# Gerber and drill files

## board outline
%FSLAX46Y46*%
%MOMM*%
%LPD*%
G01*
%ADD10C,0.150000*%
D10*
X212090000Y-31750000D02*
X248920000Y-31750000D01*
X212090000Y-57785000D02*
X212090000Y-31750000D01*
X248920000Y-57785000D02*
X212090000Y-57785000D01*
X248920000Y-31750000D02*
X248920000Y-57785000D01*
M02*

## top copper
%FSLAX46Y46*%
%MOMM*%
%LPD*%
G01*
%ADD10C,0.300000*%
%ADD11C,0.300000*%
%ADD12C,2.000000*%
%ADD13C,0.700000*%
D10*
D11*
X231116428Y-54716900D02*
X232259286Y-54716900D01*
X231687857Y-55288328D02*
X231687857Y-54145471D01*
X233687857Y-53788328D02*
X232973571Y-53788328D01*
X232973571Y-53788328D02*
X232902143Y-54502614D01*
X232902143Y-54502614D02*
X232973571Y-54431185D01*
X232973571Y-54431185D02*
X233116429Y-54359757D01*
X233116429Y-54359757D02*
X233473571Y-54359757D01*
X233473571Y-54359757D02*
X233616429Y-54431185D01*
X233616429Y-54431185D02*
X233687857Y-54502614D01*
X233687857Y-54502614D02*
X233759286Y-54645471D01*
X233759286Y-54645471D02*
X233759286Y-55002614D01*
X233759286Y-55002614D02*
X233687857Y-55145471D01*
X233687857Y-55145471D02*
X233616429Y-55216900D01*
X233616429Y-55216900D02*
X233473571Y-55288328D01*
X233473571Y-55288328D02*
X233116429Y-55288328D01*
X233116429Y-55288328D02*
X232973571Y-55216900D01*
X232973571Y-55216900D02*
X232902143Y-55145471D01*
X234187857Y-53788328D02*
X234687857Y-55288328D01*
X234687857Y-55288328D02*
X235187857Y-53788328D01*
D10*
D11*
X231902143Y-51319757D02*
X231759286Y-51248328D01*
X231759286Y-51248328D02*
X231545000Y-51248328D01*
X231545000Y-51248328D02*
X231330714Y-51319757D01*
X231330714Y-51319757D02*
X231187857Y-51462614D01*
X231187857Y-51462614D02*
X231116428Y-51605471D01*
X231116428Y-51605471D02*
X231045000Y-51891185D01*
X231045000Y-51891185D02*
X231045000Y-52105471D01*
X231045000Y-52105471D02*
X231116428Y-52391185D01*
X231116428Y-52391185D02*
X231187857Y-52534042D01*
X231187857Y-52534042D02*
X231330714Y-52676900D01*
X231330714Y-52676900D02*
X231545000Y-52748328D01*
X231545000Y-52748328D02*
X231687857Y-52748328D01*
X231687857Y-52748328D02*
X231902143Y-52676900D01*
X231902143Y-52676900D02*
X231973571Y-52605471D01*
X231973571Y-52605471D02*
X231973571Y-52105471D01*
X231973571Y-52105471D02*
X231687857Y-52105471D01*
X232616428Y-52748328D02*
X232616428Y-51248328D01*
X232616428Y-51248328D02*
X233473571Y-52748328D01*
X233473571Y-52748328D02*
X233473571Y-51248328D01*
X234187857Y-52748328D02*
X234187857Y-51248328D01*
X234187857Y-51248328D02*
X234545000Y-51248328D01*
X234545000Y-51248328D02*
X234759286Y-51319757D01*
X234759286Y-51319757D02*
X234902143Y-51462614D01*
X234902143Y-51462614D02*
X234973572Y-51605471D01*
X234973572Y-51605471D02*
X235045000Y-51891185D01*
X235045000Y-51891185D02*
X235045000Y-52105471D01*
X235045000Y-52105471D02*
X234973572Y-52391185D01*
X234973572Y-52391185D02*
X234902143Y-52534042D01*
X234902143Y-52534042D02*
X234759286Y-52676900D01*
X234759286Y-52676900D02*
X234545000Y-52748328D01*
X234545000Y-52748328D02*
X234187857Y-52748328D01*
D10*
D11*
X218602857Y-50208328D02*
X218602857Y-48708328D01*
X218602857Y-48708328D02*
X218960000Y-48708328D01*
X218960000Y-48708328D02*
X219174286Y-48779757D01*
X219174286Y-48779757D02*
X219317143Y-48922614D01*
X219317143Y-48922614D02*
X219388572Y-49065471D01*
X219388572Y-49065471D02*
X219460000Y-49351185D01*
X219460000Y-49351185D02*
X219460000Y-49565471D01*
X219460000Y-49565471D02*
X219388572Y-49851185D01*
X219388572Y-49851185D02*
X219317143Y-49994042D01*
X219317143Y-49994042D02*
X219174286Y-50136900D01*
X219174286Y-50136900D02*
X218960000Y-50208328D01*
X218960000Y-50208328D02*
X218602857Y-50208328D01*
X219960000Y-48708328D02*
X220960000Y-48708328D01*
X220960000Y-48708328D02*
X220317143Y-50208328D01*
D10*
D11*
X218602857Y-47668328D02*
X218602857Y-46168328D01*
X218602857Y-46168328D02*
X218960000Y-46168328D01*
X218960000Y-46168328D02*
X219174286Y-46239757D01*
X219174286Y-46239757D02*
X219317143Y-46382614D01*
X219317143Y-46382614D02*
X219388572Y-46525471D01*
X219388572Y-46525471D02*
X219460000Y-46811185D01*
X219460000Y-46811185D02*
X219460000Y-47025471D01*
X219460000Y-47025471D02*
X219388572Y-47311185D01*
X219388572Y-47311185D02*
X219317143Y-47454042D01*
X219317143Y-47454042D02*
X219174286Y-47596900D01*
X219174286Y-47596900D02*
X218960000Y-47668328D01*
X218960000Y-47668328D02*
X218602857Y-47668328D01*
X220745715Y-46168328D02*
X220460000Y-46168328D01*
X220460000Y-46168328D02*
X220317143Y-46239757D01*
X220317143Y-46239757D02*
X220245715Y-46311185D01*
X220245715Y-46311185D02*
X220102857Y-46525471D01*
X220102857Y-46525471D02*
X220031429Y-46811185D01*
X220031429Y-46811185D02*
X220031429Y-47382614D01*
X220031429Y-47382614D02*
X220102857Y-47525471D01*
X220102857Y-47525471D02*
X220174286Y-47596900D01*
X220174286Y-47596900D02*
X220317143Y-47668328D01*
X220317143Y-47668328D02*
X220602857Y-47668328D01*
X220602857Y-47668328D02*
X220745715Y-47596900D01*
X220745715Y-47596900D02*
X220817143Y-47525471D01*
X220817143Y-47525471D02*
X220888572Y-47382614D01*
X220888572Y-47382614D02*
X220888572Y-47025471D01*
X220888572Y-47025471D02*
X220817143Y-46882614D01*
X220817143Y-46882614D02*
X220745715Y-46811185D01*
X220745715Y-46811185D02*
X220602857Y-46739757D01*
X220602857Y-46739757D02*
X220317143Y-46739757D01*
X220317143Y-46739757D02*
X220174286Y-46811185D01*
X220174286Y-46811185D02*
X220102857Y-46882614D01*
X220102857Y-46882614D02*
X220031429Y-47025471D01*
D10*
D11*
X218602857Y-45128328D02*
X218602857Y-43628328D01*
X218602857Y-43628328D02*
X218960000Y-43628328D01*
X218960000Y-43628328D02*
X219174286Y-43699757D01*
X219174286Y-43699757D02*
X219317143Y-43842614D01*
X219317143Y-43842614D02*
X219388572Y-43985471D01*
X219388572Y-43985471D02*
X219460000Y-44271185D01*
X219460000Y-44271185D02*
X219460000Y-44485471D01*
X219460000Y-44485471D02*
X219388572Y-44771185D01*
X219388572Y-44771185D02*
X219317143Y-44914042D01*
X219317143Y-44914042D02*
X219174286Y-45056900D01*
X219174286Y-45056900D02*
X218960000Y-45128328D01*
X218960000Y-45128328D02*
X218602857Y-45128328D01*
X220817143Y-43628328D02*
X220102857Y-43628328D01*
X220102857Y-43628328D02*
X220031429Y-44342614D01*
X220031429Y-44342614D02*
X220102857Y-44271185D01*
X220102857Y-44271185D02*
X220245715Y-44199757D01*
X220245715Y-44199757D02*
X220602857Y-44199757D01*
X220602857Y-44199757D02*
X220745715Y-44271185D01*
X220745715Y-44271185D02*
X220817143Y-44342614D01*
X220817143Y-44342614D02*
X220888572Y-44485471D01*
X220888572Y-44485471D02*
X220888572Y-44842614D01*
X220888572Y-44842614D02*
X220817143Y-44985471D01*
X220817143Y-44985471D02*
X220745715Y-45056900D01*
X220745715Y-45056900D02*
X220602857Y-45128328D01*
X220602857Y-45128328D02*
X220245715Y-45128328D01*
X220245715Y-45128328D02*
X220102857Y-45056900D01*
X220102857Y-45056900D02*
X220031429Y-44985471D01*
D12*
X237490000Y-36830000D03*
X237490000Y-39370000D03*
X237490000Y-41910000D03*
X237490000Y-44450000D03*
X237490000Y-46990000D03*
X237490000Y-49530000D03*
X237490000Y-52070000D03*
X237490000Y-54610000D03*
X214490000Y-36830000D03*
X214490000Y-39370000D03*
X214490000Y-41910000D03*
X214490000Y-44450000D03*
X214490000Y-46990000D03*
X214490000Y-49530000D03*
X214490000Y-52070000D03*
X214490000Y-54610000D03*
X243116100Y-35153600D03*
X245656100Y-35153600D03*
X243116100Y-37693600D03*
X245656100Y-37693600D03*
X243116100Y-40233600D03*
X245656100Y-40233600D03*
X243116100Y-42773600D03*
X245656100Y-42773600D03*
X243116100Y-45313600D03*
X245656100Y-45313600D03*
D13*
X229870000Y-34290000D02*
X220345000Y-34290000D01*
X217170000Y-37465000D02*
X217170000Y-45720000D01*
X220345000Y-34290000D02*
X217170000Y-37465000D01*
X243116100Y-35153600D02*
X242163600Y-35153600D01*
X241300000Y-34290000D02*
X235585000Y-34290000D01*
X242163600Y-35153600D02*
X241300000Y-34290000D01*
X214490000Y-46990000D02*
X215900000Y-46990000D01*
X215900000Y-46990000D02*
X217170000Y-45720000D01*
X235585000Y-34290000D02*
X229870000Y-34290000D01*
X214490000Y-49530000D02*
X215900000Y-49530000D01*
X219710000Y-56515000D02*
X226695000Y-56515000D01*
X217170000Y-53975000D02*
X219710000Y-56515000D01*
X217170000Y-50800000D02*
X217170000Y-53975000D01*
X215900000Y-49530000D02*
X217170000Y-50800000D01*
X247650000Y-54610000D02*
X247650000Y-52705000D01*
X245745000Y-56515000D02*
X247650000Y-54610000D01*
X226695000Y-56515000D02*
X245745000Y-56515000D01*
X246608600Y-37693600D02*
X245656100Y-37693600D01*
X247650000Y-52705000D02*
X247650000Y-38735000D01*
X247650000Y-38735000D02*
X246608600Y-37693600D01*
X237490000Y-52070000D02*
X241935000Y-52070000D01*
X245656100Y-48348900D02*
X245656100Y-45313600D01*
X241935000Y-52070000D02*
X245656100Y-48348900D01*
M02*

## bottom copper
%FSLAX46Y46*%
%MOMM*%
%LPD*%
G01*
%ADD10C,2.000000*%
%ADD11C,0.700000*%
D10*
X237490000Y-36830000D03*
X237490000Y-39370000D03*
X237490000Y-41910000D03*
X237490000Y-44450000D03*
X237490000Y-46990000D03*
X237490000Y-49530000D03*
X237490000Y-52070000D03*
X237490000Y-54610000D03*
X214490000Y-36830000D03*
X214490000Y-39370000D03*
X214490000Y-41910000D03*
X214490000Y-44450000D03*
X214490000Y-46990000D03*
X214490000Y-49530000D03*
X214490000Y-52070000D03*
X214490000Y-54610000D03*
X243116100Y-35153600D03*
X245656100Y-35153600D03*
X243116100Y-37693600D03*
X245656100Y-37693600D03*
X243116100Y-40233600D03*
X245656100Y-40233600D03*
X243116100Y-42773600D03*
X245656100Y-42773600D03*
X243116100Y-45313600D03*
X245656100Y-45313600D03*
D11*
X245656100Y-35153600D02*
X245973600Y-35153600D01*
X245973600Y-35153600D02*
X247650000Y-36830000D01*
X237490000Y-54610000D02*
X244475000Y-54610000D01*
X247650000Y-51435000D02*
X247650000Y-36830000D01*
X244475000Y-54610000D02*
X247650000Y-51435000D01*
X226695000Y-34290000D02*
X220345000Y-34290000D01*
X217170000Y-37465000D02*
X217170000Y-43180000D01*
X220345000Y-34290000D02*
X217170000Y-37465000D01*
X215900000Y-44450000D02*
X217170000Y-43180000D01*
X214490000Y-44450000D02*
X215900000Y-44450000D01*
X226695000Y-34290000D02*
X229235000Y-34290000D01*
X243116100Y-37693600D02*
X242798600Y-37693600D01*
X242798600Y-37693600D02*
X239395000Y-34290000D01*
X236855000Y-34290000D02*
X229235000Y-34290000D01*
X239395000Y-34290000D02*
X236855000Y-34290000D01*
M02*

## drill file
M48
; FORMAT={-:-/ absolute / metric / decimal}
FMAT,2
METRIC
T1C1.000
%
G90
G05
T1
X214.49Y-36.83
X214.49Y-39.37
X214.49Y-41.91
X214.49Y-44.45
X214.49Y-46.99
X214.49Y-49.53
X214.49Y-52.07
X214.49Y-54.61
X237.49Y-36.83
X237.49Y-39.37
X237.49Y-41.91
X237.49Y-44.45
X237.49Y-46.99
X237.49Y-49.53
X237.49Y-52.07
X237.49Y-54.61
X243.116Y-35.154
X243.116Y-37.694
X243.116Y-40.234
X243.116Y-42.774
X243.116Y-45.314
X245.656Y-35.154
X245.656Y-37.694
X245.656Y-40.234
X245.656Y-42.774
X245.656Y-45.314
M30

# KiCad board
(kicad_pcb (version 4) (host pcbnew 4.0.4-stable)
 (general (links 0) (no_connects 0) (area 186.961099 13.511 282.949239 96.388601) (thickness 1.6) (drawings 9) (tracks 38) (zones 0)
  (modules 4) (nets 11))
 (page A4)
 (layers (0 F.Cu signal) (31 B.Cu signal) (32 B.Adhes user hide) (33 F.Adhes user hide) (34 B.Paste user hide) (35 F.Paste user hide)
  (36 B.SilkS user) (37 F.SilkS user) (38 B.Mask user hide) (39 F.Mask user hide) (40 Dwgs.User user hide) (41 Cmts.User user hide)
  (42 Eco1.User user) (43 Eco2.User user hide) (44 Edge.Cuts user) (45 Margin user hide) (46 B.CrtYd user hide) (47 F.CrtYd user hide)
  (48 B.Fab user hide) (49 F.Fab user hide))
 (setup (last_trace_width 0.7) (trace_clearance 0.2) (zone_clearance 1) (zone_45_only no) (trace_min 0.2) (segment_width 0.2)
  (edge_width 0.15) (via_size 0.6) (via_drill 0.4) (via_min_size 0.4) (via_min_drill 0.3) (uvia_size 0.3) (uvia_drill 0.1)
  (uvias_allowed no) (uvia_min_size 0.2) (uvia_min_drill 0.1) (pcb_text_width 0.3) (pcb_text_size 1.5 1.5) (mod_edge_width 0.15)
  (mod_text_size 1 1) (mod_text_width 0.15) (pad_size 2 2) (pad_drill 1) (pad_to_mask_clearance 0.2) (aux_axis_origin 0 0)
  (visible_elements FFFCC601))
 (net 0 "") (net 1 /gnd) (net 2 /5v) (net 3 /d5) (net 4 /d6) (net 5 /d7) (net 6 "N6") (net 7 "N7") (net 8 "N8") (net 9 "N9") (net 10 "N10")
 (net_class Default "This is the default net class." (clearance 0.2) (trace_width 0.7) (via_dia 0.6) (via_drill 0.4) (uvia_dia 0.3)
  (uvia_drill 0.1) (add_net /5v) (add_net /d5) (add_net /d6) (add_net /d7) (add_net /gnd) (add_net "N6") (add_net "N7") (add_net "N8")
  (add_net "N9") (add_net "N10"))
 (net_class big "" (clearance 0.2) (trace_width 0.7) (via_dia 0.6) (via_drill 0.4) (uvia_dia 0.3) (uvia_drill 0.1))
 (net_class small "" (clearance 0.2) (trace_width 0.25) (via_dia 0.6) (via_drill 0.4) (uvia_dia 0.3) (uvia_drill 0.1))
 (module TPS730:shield (layer F.Cu) (at 237.49 36.83)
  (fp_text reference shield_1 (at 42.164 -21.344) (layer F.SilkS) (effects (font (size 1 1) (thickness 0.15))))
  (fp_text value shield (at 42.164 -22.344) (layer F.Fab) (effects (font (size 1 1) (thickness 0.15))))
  (pad 14 thru_hole circle (at 0 0) (size 2 2) (drill 1) (layers *.Cu *.Mask))
  (pad 13 thru_hole circle (at 0 2.54) (size 2 2) (drill 1) (layers *.Cu *.Mask))
  (pad 12 thru_hole circle (at 0 5.08) (size 2 2) (drill 1) (layers *.Cu *.Mask))
  (pad 8 thru_hole circle (at 0 7.62) (size 2 2) (drill 1) (layers *.Cu *.Mask))
  (pad 7 thru_hole circle (at 0 10.16) (size 2 2) (drill 1) (layers *.Cu *.Mask))
  (pad 6 thru_hole circle (at 0 12.7) (size 2 2) (drill 1) (layers *.Cu *.Mask))
  (pad 5 thru_hole circle (at 0 15.24) (size 2 2) (drill 1) (layers *.Cu *.Mask) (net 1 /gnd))
  (pad 1 thru_hole circle (at 0 17.78) (size 2 2) (drill 1) (layers *.Cu *.Mask) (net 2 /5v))
  (pad 9 thru_hole circle (at -23 0) (size 2 2) (drill 1) (layers *.Cu *.Mask))
  (pad 10 thru_hole circle (at -23 2.54) (size 2 2) (drill 1) (layers *.Cu *.Mask))
  (pad 11 thru_hole circle (at -23 5.08) (size 2 2) (drill 1) (layers *.Cu *.Mask))
  (pad 4 thru_hole circle (at -23 7.62) (size 2 2) (drill 1) (layers *.Cu *.Mask) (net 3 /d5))
  (pad 3 thru_hole circle (at -23 10.16) (size 2 2) (drill 1) (layers *.Cu *.Mask) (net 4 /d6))
  (pad 2 thru_hole circle (at -23 12.7) (size 2 2) (drill 1) (layers *.Cu *.Mask) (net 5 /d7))
  (pad 15 thru_hole circle (at -23 15.24) (size 2 2) (drill 1) (layers *.Cu *.Mask))
  (pad 16 thru_hole circle (at -23 17.78) (size 2 2) (drill 1) (layers *.Cu *.Mask)))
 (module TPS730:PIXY (layer F.Cu) (at 250.7361 30.0736)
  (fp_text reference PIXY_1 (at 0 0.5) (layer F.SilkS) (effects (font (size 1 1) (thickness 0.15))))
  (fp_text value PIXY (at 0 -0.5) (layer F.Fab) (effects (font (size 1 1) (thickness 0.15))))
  (pad 1 thru_hole circle (at -7.62 5.08) (size 2 2) (drill 1) (layers *.Cu *.Mask) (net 4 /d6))
  (pad 2 thru_hole circle (at -5.08 5.08) (size 2 2) (drill 1) (layers *.Cu *.Mask) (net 2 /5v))
  (pad 3 thru_hole circle (at -7.62 7.62) (size 2 2) (drill 1) (layers *.Cu *.Mask) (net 3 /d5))
  (pad 4 thru_hole circle (at -5.08 7.62) (size 2 2) (drill 1) (layers *.Cu *.Mask) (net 5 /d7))
  (pad 5 thru_hole circle (at -7.62 10.16) (size 2 2) (drill 1) (layers *.Cu *.Mask) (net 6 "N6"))
  (pad 6 thru_hole circle (at -5.08 10.16) (size 2 2) (drill 1) (layers *.Cu *.Mask) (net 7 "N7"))
  (pad 7 thru_hole circle (at -7.62 12.7) (size 2 2) (drill 1) (layers *.Cu *.Mask) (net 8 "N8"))
  (pad 8 thru_hole circle (at -5.08 12.7) (size 2 2) (drill 1) (layers *.Cu *.Mask) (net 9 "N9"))
  (pad 9 thru_hole circle (at -7.62 15.24) (size 2 2) (drill 1) (layers *.Cu *.Mask) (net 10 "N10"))
  (pad 10 thru_hole circle (at -5.08 15.24) (size 2 2) (drill 1) (layers *.Cu *.Mask) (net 1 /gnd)))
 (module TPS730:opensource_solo (layer B.Cu) (at 227.33 44.45 180)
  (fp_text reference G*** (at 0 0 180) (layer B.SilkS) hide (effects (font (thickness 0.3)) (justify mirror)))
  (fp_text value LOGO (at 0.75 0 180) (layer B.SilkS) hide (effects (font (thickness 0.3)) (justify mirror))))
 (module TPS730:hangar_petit (layer F.Cu) (at 227.33 43.18 90)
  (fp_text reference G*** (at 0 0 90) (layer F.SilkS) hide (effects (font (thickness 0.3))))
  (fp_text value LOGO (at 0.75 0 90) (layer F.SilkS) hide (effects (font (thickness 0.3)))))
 (gr_line (start 212.09 31.75) (end 248.92 31.75) (angle 90) (layer Edge.Cuts) (width 0.15))
 (gr_line (start 212.09 57.785) (end 212.09 31.75) (angle 90) (layer Edge.Cuts) (width 0.15))
 (gr_line (start 248.92 57.785) (end 212.09 57.785) (angle 90) (layer Edge.Cuts) (width 0.15))
 (gr_line (start 248.92 31.75) (end 248.92 57.785) (angle 90) (layer Edge.Cuts) (width 0.15))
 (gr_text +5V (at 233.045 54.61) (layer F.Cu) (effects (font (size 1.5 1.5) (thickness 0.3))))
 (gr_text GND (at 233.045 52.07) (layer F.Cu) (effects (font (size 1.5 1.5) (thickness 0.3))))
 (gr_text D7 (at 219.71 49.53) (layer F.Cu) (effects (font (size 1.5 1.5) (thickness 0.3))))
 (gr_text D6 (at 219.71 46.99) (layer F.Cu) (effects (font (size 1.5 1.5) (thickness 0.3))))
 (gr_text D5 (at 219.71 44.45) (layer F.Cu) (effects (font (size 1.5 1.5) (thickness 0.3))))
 (segment (start 229.87 34.29) (end 220.345 34.29) (width 0.7) (layer F.Cu) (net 4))
 (segment (start 217.17 37.465) (end 217.17 45.72) (width 0.7) (layer F.Cu) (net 4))
 (segment (start 220.345 34.29) (end 217.17 37.465) (width 0.7) (layer F.Cu) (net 4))
 (segment (start 243.1161 35.1536) (end 242.1636 35.1536) (width 0.7) (layer F.Cu) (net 4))
 (segment (start 241.3 34.29) (end 235.585 34.29) (width 0.7) (layer F.Cu) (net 4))
 (segment (start 242.1636 35.1536) (end 241.3 34.29) (width 0.7) (layer F.Cu) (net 4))
 (segment (start 214.49 46.99) (end 215.9 46.99) (width 0.7) (layer F.Cu) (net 4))
 (segment (start 215.9 46.99) (end 217.17 45.72) (width 0.7) (layer F.Cu) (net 4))
 (segment (start 235.585 34.29) (end 229.87 34.29) (width 0.7) (layer F.Cu) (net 4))
 (segment (start 245.6561 35.1536) (end 245.9736 35.1536) (width 0.7) (layer B.Cu) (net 2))
 (segment (start 245.9736 35.1536) (end 247.65 36.83) (width 0.7) (layer B.Cu) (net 2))
 (segment (start 237.49 54.61) (end 244.475 54.61) (width 0.7) (layer B.Cu) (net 2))
 (segment (start 247.65 51.435) (end 247.65 36.83) (width 0.7) (layer B.Cu) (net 2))
 (segment (start 244.475 54.61) (end 247.65 51.435) (width 0.7) (layer B.Cu) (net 2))
 (segment (start 226.695 34.29) (end 220.345 34.29) (width 0.7) (layer B.Cu) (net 3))
 (segment (start 217.17 37.465) (end 217.17 43.18) (width 0.7) (layer B.Cu) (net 3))
 (segment (start 220.345 34.29) (end 217.17 37.465) (width 0.7) (layer B.Cu) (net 3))
 (segment (start 215.9 44.45) (end 217.17 43.18) (width 0.7) (layer B.Cu) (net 3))
 (segment (start 214.49 44.45) (end 215.9 44.45) (width 0.7) (layer B.Cu) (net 3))
 (segment (start 226.695 34.29) (end 229.235 34.29) (width 0.7) (layer B.Cu) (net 3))
 (segment (start 243.1161 37.6936) (end 242.7986 37.6936) (width 0.7) (layer B.Cu) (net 3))
 (segment (start 242.7986 37.6936) (end 239.395 34.29) (width 0.7) (layer B.Cu) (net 3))
 (segment (start 236.855 34.29) (end 229.235 34.29) (width 0.7) (layer B.Cu) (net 3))
 (segment (start 239.395 34.29) (end 236.855 34.29) (width 0.7) (layer B.Cu) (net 3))
 (segment (start 214.49 49.53) (end 215.9 49.53) (width 0.7) (layer F.Cu) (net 5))
 (segment (start 219.71 56.515) (end 226.695 56.515) (width 0.7) (layer F.Cu) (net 5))
 (segment (start 217.17 53.975) (end 219.71 56.515) (width 0.7) (layer F.Cu) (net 5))
 (segment (start 217.17 50.8) (end 217.17 53.975) (width 0.7) (layer F.Cu) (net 5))
 (segment (start 215.9 49.53) (end 217.17 50.8) (width 0.7) (layer F.Cu) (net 5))
 (segment (start 247.65 54.61) (end 247.65 52.705) (width 0.7) (layer F.Cu) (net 5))
 (segment (start 245.745 56.515) (end 247.65 54.61) (width 0.7) (layer F.Cu) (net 5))
 (segment (start 226.695 56.515) (end 245.745 56.515) (width 0.7) (layer F.Cu) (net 5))
 (segment (start 246.6086 37.6936) (end 245.6561 37.6936) (width 0.7) (layer F.Cu) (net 5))
 (segment (start 247.65 52.705) (end 247.65 38.735) (width 0.7) (layer F.Cu) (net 5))
 (segment (start 247.65 38.735) (end 246.6086 37.6936) (width 0.7) (layer F.Cu) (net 5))
 (segment (start 237.49 52.07) (end 241.935 52.07) (width 0.7) (layer F.Cu) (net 1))
 (segment (start 245.6561 48.3489) (end 245.6561 45.3136) (width 0.7) (layer F.Cu) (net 1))
 (segment (start 241.935 52.07) (end 245.6561 48.3489) (width 0.7) (layer F.Cu) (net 1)))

